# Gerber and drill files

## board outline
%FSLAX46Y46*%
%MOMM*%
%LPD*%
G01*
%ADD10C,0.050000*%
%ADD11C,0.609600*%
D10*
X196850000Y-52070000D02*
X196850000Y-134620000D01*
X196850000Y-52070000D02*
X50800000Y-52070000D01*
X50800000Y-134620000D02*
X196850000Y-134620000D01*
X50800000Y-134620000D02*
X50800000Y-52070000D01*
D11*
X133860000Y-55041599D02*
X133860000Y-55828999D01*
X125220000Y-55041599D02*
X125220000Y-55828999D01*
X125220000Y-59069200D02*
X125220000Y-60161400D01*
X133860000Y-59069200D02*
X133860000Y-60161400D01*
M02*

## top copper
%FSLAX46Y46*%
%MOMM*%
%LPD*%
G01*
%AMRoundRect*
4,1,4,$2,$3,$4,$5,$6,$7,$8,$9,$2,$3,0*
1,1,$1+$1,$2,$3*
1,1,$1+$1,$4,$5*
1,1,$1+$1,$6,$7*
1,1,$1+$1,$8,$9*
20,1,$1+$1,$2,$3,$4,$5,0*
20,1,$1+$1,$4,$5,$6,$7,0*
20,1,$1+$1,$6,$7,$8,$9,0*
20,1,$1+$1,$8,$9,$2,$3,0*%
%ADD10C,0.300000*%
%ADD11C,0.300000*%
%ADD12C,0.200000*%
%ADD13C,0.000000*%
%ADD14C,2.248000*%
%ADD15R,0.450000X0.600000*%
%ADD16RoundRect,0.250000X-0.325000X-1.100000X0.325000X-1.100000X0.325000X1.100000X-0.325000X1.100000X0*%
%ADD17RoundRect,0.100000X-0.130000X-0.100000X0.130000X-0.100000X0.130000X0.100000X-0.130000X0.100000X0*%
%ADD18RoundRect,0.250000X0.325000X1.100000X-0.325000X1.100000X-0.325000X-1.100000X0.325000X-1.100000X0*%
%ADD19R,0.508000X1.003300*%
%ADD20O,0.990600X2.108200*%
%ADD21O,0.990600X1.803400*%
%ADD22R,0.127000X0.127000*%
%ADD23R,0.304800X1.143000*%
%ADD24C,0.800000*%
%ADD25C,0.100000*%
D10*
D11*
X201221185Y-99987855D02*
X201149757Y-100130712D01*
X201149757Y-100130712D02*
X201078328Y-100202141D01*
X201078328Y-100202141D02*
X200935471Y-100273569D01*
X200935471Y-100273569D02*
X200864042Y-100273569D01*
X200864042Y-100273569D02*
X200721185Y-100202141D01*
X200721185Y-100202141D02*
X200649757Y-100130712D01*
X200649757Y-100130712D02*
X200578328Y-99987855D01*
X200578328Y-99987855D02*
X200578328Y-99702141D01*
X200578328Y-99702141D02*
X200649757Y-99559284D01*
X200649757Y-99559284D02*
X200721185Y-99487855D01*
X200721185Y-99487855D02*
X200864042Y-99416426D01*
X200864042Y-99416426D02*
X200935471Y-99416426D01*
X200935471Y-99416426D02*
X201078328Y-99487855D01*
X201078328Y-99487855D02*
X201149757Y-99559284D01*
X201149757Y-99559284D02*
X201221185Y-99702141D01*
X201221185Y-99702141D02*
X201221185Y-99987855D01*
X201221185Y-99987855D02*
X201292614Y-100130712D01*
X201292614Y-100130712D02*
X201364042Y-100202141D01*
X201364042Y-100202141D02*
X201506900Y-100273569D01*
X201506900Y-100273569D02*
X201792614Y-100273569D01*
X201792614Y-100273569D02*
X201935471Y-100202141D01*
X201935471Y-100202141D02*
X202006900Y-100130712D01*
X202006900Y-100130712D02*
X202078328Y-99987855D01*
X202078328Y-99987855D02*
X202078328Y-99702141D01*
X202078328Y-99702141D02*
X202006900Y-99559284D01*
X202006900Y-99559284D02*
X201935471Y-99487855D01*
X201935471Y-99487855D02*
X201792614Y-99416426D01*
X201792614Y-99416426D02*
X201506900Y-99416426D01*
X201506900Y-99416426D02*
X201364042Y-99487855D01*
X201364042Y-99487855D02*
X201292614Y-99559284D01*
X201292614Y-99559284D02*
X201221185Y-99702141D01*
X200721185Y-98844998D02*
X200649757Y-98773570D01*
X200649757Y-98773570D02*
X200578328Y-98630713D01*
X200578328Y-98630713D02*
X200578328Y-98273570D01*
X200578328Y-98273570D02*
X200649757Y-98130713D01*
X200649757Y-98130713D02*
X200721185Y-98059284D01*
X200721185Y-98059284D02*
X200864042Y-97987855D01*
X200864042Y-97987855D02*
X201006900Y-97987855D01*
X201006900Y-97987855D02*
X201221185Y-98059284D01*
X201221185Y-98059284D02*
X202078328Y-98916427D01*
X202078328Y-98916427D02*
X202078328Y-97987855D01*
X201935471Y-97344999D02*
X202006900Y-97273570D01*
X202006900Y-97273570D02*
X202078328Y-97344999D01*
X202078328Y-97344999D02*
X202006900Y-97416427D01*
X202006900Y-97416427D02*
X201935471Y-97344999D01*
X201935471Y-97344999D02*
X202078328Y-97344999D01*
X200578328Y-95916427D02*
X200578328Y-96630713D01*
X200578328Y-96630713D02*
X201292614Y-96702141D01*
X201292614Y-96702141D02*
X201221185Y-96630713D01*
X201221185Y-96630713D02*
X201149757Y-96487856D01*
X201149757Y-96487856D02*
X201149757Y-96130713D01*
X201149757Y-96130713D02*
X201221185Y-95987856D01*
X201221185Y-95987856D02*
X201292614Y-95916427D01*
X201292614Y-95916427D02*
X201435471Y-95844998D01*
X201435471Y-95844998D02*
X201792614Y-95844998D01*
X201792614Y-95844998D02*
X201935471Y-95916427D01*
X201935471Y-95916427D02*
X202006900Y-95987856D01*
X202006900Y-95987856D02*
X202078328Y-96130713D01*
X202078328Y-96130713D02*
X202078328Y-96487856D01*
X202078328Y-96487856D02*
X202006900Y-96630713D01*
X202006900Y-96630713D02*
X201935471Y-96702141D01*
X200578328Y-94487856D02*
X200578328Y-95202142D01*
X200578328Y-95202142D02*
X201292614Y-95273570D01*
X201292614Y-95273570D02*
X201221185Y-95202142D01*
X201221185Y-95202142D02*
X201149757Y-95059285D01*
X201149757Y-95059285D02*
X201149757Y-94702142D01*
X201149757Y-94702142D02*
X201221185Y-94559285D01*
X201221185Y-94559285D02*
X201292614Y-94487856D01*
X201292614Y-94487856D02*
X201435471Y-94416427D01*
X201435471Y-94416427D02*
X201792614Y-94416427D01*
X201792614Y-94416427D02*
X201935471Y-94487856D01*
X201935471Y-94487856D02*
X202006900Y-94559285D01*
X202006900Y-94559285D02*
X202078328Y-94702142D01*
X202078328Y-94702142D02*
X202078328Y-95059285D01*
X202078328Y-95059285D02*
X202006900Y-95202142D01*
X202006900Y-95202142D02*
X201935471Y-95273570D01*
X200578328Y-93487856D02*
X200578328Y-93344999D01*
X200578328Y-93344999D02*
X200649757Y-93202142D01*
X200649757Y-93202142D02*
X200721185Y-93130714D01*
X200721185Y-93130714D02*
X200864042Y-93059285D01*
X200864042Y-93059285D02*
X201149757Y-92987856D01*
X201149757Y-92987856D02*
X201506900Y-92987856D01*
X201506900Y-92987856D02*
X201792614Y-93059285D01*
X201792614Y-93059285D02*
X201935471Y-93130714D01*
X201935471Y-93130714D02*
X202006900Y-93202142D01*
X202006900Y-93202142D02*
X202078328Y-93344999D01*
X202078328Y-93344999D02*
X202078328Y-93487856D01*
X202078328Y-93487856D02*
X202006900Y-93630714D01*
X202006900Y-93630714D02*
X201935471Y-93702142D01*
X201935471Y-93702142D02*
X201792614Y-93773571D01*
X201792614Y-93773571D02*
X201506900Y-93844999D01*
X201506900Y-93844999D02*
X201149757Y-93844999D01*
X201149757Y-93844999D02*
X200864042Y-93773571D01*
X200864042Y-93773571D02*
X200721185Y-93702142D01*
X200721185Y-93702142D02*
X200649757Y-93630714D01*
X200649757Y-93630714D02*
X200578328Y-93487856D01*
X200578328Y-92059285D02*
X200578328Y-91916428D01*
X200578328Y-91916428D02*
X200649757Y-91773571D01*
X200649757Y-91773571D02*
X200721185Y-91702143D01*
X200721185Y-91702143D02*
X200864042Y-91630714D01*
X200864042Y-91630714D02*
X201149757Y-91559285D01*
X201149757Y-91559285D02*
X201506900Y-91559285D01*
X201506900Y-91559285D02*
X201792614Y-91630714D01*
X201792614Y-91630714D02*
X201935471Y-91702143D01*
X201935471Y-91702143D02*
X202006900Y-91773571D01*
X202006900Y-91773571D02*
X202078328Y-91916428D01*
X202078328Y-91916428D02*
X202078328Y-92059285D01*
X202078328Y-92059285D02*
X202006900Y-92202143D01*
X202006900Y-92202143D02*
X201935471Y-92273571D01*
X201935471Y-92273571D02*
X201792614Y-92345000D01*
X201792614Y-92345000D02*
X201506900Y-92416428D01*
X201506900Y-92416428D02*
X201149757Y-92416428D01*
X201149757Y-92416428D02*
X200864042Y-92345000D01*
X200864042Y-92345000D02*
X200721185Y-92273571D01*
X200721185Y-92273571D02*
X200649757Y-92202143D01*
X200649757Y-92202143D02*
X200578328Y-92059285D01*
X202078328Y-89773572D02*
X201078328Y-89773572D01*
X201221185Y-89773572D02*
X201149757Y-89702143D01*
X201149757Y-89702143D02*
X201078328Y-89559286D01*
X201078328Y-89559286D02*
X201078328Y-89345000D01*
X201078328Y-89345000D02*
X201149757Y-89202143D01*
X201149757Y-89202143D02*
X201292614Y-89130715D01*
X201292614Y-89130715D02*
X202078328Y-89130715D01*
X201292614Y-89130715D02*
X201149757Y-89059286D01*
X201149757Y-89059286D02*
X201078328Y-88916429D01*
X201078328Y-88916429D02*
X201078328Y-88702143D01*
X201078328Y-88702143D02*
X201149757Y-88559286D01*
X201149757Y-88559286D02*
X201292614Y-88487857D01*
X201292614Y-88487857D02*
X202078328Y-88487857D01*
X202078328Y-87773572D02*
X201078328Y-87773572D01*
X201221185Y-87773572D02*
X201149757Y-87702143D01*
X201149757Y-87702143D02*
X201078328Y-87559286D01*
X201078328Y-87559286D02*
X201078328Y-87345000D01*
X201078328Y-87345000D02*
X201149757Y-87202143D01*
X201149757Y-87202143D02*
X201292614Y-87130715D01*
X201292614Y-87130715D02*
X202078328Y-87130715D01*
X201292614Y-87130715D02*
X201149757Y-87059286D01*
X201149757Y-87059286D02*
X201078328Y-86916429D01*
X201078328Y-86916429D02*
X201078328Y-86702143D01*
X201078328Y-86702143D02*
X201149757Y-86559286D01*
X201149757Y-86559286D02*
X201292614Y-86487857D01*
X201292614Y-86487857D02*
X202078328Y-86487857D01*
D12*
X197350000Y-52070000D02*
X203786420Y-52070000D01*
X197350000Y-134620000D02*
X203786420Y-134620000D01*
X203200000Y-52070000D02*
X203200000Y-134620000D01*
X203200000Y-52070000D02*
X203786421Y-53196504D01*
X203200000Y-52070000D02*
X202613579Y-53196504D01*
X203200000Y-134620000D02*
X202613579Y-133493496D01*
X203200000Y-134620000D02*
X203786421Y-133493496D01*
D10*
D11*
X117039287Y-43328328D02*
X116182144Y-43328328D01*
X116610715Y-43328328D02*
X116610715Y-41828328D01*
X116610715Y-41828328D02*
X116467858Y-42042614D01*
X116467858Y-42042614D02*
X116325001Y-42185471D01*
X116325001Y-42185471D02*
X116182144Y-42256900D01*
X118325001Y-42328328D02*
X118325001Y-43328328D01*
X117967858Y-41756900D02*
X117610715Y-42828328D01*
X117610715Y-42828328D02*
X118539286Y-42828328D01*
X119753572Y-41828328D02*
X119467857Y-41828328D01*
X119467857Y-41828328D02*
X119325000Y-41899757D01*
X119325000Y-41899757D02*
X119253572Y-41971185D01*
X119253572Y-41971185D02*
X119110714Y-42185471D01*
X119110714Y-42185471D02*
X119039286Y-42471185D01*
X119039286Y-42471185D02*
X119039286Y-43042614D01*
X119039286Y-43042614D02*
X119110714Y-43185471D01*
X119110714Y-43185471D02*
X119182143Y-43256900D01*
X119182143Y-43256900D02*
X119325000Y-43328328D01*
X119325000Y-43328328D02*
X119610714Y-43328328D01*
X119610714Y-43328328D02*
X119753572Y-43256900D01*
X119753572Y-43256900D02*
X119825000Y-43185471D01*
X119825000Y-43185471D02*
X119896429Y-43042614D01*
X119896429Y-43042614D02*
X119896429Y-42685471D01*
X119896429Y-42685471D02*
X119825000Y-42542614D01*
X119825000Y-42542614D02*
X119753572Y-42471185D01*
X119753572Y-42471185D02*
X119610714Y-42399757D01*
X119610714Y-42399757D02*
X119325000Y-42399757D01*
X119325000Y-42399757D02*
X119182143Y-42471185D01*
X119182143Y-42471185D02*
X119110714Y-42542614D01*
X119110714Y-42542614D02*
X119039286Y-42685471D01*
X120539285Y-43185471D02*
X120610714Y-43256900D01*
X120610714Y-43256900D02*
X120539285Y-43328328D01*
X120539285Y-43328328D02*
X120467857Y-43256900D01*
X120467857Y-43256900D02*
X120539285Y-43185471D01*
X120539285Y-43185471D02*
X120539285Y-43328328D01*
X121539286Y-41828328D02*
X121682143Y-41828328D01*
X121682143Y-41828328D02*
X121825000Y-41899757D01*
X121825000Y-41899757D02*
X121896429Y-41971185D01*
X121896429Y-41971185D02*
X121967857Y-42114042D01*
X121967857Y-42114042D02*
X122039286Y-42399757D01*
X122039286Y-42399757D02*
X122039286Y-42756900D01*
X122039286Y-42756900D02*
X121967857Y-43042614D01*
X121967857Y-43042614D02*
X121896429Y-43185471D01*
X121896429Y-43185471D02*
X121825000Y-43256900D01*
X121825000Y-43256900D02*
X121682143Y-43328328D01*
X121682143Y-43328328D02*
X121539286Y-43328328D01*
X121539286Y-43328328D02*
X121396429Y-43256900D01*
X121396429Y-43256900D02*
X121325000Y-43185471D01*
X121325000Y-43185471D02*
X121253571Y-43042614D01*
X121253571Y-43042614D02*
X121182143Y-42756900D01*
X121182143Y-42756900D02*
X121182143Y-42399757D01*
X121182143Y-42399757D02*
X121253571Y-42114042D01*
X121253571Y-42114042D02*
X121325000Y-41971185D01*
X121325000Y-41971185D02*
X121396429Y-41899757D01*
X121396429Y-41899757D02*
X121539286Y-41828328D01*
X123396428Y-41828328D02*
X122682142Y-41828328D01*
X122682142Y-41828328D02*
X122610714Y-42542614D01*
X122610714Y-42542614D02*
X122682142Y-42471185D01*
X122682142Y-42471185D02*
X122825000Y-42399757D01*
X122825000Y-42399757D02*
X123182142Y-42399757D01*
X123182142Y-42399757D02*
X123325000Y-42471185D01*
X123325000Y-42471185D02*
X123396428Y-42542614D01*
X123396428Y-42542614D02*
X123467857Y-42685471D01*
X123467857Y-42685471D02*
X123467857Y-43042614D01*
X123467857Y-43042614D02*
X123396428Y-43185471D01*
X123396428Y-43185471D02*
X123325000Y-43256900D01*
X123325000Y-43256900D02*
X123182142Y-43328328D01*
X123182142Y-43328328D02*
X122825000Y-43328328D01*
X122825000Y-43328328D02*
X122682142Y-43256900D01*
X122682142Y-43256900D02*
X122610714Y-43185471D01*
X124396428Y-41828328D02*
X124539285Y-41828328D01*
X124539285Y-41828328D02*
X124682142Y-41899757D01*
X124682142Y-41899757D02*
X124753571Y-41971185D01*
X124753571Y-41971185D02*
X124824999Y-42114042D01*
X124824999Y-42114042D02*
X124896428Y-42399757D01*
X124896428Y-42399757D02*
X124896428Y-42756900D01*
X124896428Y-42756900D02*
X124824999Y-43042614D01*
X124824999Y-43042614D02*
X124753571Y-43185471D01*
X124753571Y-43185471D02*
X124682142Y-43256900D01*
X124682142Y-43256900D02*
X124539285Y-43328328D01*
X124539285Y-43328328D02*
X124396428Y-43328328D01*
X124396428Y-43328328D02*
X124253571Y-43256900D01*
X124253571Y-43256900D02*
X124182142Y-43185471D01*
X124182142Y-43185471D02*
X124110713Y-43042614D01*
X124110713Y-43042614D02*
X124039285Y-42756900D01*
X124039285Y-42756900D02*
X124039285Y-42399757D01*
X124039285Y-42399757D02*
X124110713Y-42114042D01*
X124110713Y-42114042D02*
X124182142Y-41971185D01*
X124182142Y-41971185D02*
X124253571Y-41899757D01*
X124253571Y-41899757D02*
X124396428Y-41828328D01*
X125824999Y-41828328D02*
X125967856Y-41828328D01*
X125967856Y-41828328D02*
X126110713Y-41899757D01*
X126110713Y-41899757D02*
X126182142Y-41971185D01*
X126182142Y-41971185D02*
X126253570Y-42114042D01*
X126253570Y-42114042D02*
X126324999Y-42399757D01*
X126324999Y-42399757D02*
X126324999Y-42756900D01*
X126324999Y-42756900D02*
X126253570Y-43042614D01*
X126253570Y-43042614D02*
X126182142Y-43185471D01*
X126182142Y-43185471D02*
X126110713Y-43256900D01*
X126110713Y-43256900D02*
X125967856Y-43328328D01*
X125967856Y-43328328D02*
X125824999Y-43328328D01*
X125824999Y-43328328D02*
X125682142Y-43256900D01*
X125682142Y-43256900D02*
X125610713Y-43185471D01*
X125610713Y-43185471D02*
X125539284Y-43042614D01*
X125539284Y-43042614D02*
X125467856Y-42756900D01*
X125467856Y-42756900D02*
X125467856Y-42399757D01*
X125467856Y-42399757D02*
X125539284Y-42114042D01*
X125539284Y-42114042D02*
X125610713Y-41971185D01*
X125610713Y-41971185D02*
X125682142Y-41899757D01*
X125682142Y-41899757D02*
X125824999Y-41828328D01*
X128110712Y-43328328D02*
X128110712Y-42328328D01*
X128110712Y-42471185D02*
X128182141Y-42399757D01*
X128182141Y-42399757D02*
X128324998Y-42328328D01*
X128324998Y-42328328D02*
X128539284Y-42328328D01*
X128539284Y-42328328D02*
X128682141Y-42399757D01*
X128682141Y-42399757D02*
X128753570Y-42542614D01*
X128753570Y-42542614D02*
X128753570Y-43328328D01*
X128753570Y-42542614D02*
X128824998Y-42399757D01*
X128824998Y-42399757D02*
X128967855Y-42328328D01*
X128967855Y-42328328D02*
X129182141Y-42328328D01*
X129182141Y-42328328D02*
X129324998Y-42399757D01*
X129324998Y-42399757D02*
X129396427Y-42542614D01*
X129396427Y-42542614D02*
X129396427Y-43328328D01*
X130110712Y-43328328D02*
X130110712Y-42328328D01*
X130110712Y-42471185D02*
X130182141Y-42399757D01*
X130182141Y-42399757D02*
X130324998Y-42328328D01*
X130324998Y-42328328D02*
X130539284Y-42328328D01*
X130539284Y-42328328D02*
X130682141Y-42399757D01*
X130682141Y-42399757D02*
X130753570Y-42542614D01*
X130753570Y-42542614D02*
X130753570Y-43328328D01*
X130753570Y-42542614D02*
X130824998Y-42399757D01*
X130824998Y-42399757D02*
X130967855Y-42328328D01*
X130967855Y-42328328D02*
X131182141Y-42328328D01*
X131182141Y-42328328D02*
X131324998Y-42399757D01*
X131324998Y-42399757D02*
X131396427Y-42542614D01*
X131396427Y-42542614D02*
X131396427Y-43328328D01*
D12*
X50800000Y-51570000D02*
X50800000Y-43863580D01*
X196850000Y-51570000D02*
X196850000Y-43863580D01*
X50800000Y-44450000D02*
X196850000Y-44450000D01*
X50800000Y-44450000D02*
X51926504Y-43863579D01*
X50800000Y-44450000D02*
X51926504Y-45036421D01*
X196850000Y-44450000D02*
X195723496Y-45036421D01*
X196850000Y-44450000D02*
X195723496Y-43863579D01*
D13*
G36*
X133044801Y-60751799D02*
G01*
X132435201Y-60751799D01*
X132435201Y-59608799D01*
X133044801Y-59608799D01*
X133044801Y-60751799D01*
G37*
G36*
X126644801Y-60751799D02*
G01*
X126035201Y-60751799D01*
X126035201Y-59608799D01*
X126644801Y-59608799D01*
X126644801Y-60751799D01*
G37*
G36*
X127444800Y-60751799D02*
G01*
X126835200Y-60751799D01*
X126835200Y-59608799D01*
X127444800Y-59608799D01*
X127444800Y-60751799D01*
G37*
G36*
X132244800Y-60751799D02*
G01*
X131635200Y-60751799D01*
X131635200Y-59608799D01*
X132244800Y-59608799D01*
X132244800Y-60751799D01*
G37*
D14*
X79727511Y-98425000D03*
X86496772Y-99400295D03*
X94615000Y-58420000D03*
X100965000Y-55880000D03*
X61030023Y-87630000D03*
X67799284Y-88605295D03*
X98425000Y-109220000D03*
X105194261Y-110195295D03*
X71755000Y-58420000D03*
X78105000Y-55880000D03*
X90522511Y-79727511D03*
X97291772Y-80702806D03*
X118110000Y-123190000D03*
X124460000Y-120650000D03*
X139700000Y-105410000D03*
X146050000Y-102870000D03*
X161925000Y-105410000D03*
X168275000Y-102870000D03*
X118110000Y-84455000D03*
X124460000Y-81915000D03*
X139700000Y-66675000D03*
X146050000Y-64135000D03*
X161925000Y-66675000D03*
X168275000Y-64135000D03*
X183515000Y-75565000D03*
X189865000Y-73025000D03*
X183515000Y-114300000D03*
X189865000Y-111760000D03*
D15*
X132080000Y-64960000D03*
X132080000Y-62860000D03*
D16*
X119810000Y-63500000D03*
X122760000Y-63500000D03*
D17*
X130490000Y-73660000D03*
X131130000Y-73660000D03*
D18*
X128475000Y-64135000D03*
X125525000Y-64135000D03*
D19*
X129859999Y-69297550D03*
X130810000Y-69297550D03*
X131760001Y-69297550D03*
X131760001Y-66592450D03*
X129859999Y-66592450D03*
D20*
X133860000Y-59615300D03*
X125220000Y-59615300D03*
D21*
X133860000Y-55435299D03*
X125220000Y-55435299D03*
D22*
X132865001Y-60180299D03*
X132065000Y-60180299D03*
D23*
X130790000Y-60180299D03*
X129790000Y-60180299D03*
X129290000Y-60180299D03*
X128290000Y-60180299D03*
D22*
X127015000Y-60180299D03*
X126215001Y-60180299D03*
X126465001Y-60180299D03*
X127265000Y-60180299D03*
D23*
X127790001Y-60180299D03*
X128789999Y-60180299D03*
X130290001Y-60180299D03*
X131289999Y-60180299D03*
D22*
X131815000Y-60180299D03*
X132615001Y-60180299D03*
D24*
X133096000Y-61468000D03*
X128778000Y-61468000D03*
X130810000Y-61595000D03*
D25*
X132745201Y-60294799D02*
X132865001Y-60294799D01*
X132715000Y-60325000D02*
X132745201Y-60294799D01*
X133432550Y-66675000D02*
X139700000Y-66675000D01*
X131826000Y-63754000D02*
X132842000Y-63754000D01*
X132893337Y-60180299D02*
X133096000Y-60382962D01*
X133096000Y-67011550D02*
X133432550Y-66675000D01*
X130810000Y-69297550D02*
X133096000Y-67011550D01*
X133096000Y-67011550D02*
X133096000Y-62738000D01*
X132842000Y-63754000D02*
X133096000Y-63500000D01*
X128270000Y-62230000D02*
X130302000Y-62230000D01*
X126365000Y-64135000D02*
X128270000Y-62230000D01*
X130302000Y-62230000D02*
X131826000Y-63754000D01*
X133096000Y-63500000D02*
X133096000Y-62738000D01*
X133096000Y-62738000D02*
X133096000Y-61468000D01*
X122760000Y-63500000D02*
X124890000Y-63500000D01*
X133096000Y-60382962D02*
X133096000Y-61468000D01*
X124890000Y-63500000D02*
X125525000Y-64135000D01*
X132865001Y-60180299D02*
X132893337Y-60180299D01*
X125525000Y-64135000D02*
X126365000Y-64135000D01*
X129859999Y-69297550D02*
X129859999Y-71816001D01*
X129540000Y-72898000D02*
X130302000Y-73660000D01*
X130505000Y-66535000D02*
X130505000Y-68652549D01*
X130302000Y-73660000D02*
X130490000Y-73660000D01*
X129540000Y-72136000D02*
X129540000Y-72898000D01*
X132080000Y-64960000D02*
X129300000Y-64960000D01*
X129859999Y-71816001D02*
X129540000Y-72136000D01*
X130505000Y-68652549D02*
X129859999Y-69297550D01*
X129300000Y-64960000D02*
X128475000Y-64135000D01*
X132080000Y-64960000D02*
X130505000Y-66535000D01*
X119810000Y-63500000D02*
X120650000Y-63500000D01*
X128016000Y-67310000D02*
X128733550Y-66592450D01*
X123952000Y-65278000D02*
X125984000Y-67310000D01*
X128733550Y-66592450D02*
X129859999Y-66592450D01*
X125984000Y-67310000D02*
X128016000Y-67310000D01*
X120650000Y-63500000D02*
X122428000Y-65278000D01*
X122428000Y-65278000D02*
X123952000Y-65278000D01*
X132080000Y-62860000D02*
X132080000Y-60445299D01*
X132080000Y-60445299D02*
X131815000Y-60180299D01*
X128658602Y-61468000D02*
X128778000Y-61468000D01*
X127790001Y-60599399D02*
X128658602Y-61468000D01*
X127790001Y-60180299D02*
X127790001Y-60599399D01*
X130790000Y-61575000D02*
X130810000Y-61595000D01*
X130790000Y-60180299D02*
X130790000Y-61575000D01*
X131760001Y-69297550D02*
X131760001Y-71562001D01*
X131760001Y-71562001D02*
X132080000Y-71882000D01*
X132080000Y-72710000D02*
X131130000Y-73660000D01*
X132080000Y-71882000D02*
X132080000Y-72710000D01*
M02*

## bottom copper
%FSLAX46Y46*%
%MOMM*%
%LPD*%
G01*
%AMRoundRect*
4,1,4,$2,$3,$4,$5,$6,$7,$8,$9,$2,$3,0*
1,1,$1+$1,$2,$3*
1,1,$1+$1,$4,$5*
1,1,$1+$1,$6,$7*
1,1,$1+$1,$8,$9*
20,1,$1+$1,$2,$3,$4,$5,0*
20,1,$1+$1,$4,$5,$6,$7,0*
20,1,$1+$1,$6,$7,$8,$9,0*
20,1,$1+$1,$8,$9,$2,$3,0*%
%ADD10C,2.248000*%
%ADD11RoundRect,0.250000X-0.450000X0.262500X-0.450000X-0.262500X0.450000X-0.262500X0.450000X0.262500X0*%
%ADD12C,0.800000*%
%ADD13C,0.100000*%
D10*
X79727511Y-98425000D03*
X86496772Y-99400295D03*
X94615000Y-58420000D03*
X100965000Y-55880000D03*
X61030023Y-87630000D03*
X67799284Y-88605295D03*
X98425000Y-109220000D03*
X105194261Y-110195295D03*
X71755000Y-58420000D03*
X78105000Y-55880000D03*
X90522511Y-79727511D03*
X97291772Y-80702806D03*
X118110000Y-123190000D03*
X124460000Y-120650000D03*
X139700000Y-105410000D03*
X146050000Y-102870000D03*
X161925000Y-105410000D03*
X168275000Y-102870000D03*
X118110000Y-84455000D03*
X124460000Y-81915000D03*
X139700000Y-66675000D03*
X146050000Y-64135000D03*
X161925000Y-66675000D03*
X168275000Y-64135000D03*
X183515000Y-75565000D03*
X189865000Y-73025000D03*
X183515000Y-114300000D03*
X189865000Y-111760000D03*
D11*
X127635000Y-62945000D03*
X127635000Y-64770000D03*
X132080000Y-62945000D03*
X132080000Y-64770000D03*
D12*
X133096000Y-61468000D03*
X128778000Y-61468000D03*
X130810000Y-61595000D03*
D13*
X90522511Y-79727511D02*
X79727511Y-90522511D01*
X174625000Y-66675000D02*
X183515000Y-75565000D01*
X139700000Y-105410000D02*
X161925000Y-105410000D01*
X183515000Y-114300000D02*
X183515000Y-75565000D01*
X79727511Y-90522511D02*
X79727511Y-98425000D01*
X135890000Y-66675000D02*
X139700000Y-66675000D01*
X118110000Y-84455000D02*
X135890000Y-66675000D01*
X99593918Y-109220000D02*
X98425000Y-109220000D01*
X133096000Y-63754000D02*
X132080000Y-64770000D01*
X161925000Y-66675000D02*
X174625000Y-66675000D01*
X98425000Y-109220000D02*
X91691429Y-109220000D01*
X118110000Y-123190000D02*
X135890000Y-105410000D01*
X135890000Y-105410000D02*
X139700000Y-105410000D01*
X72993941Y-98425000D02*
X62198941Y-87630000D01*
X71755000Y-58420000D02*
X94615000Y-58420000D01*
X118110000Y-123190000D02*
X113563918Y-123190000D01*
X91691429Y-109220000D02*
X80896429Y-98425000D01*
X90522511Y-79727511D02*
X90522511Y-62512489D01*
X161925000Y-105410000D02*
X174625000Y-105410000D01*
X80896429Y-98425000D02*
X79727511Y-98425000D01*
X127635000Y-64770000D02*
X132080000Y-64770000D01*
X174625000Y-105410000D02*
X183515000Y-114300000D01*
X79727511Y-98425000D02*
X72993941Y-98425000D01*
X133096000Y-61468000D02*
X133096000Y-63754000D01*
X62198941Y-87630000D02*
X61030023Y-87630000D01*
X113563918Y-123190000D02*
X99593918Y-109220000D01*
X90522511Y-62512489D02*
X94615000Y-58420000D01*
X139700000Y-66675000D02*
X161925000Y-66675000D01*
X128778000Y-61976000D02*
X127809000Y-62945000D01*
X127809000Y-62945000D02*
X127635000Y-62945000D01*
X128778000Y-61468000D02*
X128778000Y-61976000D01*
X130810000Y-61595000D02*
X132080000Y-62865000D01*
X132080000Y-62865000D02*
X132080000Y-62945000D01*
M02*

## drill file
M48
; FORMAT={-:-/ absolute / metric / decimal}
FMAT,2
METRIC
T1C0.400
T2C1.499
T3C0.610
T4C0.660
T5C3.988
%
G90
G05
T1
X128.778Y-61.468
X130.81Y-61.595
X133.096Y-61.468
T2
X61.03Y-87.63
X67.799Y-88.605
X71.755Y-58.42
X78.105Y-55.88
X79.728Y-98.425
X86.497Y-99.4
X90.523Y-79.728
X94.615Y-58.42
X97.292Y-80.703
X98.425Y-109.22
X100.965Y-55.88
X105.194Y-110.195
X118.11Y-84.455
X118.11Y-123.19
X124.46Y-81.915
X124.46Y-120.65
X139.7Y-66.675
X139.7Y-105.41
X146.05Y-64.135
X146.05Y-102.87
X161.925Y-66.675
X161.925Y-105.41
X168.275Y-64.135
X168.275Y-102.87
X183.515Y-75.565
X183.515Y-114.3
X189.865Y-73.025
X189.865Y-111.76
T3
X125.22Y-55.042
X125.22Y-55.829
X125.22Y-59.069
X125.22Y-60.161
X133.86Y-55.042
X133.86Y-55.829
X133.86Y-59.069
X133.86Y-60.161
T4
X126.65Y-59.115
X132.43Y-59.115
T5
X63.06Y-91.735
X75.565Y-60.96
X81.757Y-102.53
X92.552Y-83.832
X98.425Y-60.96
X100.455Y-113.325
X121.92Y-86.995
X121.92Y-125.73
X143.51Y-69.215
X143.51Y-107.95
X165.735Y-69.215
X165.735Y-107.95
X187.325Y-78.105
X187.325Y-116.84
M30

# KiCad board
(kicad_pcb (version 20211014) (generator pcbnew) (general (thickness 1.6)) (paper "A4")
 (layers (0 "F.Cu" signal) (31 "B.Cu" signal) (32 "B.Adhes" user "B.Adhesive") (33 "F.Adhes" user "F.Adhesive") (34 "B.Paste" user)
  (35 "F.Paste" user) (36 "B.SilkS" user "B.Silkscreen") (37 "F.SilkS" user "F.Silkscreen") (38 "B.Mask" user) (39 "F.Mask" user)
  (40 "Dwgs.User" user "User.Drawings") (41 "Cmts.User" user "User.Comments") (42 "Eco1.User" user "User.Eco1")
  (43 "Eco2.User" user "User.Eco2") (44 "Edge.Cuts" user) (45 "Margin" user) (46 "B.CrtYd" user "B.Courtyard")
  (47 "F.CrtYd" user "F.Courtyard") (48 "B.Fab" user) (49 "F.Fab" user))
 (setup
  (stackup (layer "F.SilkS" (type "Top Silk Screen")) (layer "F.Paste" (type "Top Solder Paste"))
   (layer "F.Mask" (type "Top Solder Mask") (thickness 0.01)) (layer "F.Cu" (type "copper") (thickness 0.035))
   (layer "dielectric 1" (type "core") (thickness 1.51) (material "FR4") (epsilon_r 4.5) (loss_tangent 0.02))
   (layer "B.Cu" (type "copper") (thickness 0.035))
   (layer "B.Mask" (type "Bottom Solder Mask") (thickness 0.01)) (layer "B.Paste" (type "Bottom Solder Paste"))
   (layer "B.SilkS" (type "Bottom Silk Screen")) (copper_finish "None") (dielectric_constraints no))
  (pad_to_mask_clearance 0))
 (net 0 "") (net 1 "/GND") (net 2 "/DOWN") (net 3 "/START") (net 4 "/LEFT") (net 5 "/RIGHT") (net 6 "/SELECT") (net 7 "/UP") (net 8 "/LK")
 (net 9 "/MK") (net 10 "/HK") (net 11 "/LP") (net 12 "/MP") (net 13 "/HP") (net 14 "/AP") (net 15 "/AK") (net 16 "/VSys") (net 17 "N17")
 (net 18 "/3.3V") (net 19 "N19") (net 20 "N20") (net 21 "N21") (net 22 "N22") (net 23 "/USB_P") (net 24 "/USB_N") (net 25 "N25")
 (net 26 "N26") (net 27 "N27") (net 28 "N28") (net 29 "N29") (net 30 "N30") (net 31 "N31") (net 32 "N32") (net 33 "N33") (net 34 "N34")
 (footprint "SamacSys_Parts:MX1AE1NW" (layer "F.Cu") (at 79.727511 98.425 -30)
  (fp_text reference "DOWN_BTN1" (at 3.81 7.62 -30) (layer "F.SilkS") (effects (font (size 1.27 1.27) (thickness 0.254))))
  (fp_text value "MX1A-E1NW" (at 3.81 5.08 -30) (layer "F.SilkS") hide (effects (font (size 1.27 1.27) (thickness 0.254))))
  (pad "" np_thru_hole circle (at 3.81 2.54 330) (size 3.9878 3.9878) (drill 3.9878) (layers *.Cu *.Mask))
  (pad "1" thru_hole circle (at 0 0 330) (size 2.248 2.248) (drill 1.4986) (layers *.Cu *.Mask) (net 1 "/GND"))
  (pad "2" thru_hole circle (at 6.35 -2.54 330) (size 2.248 2.248) (drill 1.4986) (layers *.Cu *.Mask) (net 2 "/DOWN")))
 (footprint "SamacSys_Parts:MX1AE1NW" (layer "F.Cu") (at 94.615 58.42)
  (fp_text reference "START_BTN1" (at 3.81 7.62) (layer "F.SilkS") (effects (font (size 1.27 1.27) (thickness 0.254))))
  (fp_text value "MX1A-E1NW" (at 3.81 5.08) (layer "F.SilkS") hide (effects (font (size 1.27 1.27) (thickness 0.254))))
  (pad "" np_thru_hole circle (at 3.81 2.54) (size 3.9878 3.9878) (drill 3.9878) (layers *.Cu *.Mask))
  (pad "1" thru_hole circle (at 0 0) (size 2.248 2.248) (drill 1.4986) (layers *.Cu *.Mask) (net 1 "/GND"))
  (pad "2" thru_hole circle (at 6.35 -2.54) (size 2.248 2.248) (drill 1.4986) (layers *.Cu *.Mask) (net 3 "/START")))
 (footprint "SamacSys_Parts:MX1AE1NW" (layer "F.Cu") (at 61.030023 87.63 -30)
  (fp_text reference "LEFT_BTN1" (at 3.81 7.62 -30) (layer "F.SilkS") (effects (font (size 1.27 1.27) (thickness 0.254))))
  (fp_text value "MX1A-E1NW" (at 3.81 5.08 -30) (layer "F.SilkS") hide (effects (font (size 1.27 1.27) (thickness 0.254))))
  (pad "" np_thru_hole circle (at 3.81 2.54 330) (size 3.9878 3.9878) (drill 3.9878) (layers *.Cu *.Mask))
  (pad "1" thru_hole circle (at 0 0 330) (size 2.248 2.248) (drill 1.4986) (layers *.Cu *.Mask) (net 1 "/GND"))
  (pad "2" thru_hole circle (at 6.35 -2.54 330) (size 2.248 2.248) (drill 1.4986) (layers *.Cu *.Mask) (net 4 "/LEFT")))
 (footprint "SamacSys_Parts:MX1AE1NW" (layer "F.Cu") (at 98.425 109.22 -30)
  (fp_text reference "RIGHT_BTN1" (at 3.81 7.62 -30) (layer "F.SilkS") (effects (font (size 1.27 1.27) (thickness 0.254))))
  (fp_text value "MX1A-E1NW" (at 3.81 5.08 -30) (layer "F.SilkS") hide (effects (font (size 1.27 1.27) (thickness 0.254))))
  (pad "" np_thru_hole circle (at 3.81 2.54 330) (size 3.9878 3.9878) (drill 3.9878) (layers *.Cu *.Mask))
  (pad "1" thru_hole circle (at 0 0 330) (size 2.248 2.248) (drill 1.4986) (layers *.Cu *.Mask) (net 1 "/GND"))
  (pad "2" thru_hole circle (at 6.35 -2.54 330) (size 2.248 2.248) (drill 1.4986) (layers *.Cu *.Mask) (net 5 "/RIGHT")))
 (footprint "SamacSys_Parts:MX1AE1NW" (layer "F.Cu") (at 71.755 58.42)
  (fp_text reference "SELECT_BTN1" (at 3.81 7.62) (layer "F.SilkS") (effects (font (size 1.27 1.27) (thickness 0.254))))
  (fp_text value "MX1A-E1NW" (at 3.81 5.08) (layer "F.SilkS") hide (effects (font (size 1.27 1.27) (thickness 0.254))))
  (pad "" np_thru_hole circle (at 3.81 2.54) (size 3.9878 3.9878) (drill 3.9878) (layers *.Cu *.Mask))
  (pad "1" thru_hole circle (at 0 0) (size 2.248 2.248) (drill 1.4986) (layers *.Cu *.Mask) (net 1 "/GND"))
  (pad "2" thru_hole circle (at 6.35 -2.54) (size 2.248 2.248) (drill 1.4986) (layers *.Cu *.Mask) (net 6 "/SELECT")))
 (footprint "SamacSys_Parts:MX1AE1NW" (layer "F.Cu") (at 90.522511 79.727511 -30)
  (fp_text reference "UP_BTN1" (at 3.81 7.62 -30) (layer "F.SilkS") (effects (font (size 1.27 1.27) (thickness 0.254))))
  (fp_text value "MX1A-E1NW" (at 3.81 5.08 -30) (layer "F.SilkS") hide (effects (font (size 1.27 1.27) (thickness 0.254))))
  (pad "" np_thru_hole circle (at 3.81 2.54 330) (size 3.9878 3.9878) (drill 3.9878) (layers *.Cu *.Mask))
  (pad "1" thru_hole circle (at 0 0 330) (size 2.248 2.248) (drill 1.4986) (layers *.Cu *.Mask) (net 1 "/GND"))
  (pad "2" thru_hole circle (at 6.35 -2.54 330) (size 2.248 2.248) (drill 1.4986) (layers *.Cu *.Mask) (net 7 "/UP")))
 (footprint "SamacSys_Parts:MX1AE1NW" (layer "F.Cu") (at 118.11 123.19)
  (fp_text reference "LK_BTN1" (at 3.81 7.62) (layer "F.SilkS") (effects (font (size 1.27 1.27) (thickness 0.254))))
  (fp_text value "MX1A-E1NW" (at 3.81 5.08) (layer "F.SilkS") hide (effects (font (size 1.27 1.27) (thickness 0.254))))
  (pad "" np_thru_hole circle (at 3.81 2.54) (size 3.9878 3.9878) (drill 3.9878) (layers *.Cu *.Mask))
  (pad "1" thru_hole circle (at 0 0) (size 2.248 2.248) (drill 1.4986) (layers *.Cu *.Mask) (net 1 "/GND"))
  (pad "2" thru_hole circle (at 6.35 -2.54) (size 2.248 2.248) (drill 1.4986) (layers *.Cu *.Mask) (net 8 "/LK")))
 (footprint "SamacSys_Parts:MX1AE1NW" (layer "F.Cu") (at 139.7 105.41)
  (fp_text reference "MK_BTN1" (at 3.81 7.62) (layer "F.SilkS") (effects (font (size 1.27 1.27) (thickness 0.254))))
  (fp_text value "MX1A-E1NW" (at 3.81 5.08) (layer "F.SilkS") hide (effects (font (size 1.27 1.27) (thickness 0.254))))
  (pad "" np_thru_hole circle (at 3.81 2.54) (size 3.9878 3.9878) (drill 3.9878) (layers *.Cu *.Mask))
  (pad "1" thru_hole circle (at 0 0) (size 2.248 2.248) (drill 1.4986) (layers *.Cu *.Mask) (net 1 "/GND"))
  (pad "2" thru_hole circle (at 6.35 -2.54) (size 2.248 2.248) (drill 1.4986) (layers *.Cu *.Mask) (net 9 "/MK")))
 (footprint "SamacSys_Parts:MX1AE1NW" (layer "F.Cu") (at 161.925 105.41)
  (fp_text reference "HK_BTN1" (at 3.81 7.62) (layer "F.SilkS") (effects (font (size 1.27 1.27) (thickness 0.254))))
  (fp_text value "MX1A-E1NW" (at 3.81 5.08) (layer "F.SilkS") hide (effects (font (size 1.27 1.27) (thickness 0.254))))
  (pad "" np_thru_hole circle (at 3.81 2.54) (size 3.9878 3.9878) (drill 3.9878) (layers *.Cu *.Mask))
  (pad "1" thru_hole circle (at 0 0) (size 2.248 2.248) (drill 1.4986) (layers *.Cu *.Mask) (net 1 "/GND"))
  (pad "2" thru_hole circle (at 6.35 -2.54) (size 2.248 2.248) (drill 1.4986) (layers *.Cu *.Mask) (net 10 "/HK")))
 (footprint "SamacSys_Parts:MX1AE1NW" (layer "F.Cu") (at 118.11 84.455)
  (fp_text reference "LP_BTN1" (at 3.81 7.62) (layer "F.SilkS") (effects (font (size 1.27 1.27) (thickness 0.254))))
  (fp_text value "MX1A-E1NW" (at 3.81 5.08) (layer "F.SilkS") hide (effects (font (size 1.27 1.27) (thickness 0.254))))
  (pad "" np_thru_hole circle (at 3.81 2.54) (size 3.9878 3.9878) (drill 3.9878) (layers *.Cu *.Mask))
  (pad "1" thru_hole circle (at 0 0) (size 2.248 2.248) (drill 1.4986) (layers *.Cu *.Mask) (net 1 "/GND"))
  (pad "2" thru_hole circle (at 6.35 -2.54) (size 2.248 2.248) (drill 1.4986) (layers *.Cu *.Mask) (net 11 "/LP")))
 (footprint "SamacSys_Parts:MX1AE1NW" (layer "F.Cu") (at 139.7 66.675)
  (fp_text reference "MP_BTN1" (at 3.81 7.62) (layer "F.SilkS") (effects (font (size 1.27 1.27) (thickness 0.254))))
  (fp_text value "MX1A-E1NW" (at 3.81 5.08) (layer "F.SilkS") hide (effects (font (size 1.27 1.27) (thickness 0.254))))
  (pad "" np_thru_hole circle (at 3.81 2.54) (size 3.9878 3.9878) (drill 3.9878) (layers *.Cu *.Mask))
  (pad "1" thru_hole circle (at 0 0) (size 2.248 2.248) (drill 1.4986) (layers *.Cu *.Mask) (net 1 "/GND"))
  (pad "2" thru_hole circle (at 6.35 -2.54) (size 2.248 2.248) (drill 1.4986) (layers *.Cu *.Mask) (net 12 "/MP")))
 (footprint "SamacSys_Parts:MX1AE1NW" (layer "F.Cu") (at 161.925 66.675)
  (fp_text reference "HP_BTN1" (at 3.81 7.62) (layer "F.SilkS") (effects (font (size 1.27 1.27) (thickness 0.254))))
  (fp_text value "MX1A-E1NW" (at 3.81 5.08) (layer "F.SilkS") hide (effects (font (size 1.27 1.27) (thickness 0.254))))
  (pad "" np_thru_hole circle (at 3.81 2.54) (size 3.9878 3.9878) (drill 3.9878) (layers *.Cu *.Mask))
  (pad "1" thru_hole circle (at 0 0) (size 2.248 2.248) (drill 1.4986) (layers *.Cu *.Mask) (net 1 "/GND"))
  (pad "2" thru_hole circle (at 6.35 -2.54) (size 2.248 2.248) (drill 1.4986) (layers *.Cu *.Mask) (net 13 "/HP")))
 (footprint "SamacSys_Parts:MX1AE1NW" (layer "F.Cu") (at 183.515 75.565)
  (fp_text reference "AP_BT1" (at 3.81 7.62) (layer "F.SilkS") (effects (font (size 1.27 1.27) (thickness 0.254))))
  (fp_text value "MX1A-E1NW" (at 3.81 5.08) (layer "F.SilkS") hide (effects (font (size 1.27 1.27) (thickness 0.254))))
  (pad "" np_thru_hole circle (at 3.81 2.54) (size 3.9878 3.9878) (drill 3.9878) (layers *.Cu *.Mask))
  (pad "1" thru_hole circle (at 0 0) (size 2.248 2.248) (drill 1.4986) (layers *.Cu *.Mask) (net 1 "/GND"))
  (pad "2" thru_hole circle (at 6.35 -2.54) (size 2.248 2.248) (drill 1.4986) (layers *.Cu *.Mask) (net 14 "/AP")))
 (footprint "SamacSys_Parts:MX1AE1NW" (layer "F.Cu") (at 183.515 114.3)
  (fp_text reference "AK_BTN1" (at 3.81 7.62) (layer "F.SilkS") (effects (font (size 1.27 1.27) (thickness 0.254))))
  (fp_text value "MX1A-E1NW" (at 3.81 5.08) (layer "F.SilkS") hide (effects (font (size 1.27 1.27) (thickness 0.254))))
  (pad "" np_thru_hole circle (at 3.81 2.54) (size 3.9878 3.9878) (drill 3.9878) (layers *.Cu *.Mask))
  (pad "1" thru_hole circle (at 0 0) (size 2.248 2.248) (drill 1.4986) (layers *.Cu *.Mask) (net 1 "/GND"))
  (pad "2" thru_hole circle (at 6.35 -2.54) (size 2.248 2.248) (drill 1.4986) (layers *.Cu *.Mask) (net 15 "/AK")))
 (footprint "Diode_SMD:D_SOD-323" (layer "F.Cu") (at 132.08 63.91 90)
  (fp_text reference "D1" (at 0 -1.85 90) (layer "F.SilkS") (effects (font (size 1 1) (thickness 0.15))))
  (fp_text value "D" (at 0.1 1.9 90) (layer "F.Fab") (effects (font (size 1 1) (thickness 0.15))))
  (pad "1" smd rect (at -1.05 0 90) (size 0.6 0.45) (layers "F.Cu" "F.Paste" "F.Mask") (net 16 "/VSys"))
  (pad "2" smd rect (at 1.05 0 90) (size 0.6 0.45) (layers "F.Cu" "F.Paste" "F.Mask") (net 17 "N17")))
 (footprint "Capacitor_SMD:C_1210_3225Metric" (layer "F.Cu") (at 121.285 63.5)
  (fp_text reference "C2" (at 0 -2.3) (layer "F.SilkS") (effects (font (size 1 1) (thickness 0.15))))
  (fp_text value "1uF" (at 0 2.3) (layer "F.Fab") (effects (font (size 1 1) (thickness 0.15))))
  (pad "1" smd roundrect (at -1.475 0) (size 1.15 2.7) (layers "F.Cu" "F.Paste" "F.Mask") (roundrect_rratio 0.217391) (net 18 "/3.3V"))
  (pad "2" smd roundrect (at 1.475 0) (size 1.15 2.7) (layers "F.Cu" "F.Paste" "F.Mask") (roundrect_rratio 0.217391) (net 1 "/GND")))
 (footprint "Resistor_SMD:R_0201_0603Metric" (layer "F.Cu") (at 130.81 73.66)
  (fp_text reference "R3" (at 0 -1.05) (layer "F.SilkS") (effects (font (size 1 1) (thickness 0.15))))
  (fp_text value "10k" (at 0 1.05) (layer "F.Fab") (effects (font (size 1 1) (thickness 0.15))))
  (pad "" smd roundrect (at -0.345 0) (size 0.318 0.36) (layers "F.Paste") (roundrect_rratio 0.25))
  (pad "" smd roundrect (at 0.345 0) (size 0.318 0.36) (layers "F.Paste") (roundrect_rratio 0.25))
  (pad "1" smd roundrect (at -0.32 0) (size 0.46 0.4) (layers "F.Cu" "F.Mask") (roundrect_rratio 0.25) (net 16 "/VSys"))
  (pad "2" smd roundrect (at 0.32 0) (size 0.46 0.4) (layers "F.Cu" "F.Mask") (roundrect_rratio 0.25) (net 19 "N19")))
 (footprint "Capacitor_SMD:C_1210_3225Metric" (layer "F.Cu") (at 127 64.135 180)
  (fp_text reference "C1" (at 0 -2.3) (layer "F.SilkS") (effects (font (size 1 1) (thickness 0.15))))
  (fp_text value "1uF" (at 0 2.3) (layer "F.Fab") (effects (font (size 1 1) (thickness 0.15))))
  (pad "1" smd roundrect (at -1.475 0 180) (size 1.15 2.7) (layers "F.Cu" "F.Paste" "F.Mask") (roundrect_rratio 0.217391) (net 16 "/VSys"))
  (pad "2" smd roundrect (at 1.475 0 180) (size 1.15 2.7) (layers "F.Cu" "F.Paste" "F.Mask") (roundrect_rratio 0.217391) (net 1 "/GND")))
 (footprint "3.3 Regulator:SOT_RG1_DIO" (layer "F.Cu") (at 130.81 67.945 90)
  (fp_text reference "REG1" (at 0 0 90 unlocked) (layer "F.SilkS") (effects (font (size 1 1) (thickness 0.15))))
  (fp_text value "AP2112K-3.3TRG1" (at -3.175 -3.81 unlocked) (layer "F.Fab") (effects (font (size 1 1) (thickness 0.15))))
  (pad "1" smd rect (at -1.35255 -0.950001 90) (size 1.0033 0.508) (layers "F.Cu" "F.Paste" "F.Mask") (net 16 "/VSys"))
  (pad "2" smd rect (at -1.35255 0 90) (size 1.0033 0.508) (layers "F.Cu" "F.Paste" "F.Mask") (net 1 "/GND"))
  (pad "3" smd rect (at -1.35255 0.950001 90) (size 1.0033 0.508) (layers "F.Cu" "F.Paste" "F.Mask") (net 19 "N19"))
  (pad "4" smd rect (at 1.35255 0.950001 90) (size 1.0033 0.508) (layers "F.Cu" "F.Paste" "F.Mask") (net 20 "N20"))
  (pad "5" smd rect (at 1.35255 -0.950001 90) (size 1.0033 0.508) (layers "F.Cu" "F.Paste" "F.Mask") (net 18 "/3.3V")))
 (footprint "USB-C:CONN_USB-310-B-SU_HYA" (layer "F.Cu") (at 129.54 56.515 180)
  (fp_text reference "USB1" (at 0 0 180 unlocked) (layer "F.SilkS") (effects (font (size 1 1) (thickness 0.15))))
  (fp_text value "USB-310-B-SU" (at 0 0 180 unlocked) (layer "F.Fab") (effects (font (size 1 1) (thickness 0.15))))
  (fp_poly
   (pts (xy -2.895201 -4.236799) (xy -3.504801 -4.236799) (xy -3.504801 -3.093799) (xy -2.895201 -3.093799)) (layer "F.Cu") (width 0)
   (fill solid))
  (fp_poly
   (pts (xy 3.504799 -4.236799) (xy 2.895199 -4.236799) (xy 2.895199 -3.093799) (xy 3.504799 -3.093799)) (layer "F.Cu") (width 0)
   (fill solid))
  (fp_poly
   (pts (xy 2.7048 -4.236799) (xy 2.0952 -4.236799) (xy 2.0952 -3.093799) (xy 2.7048 -3.093799)) (layer "F.Cu") (width 0) (fill solid))
  (fp_poly
   (pts (xy -2.0952 -4.236799) (xy -2.7048 -4.236799) (xy -2.7048 -3.093799) (xy -2.0952 -3.093799)) (layer "F.Cu") (width 0) (fill solid))
  (fp_line (start -4.32 1.473401) (end -4.32 0.686001) (layer "Edge.Cuts") (width 0.6096))
  (fp_line (start 4.32 1.473401) (end 4.32 0.686001) (layer "Edge.Cuts") (width 0.6096))
  (fp_line (start 4.32 -2.5542) (end 4.32 -3.6464) (layer "Edge.Cuts") (width 0.6096))
  (fp_line (start -4.32 -2.5542) (end -4.32 -3.6464) (layer "Edge.Cuts") (width 0.6096))
  (pad "" np_thru_hole circle (at -4.32 1.473401 180) (size 0.6096 0.6096) (drill 0.6096) (layers))
  (pad "" np_thru_hole circle (at 4.32 0.686001 180) (size 0.6096 0.6096) (drill 0.6096) (layers))
  (pad "" np_thru_hole circle (at 2.889999 -2.6003 180) (size 0.6604 0.6604) (drill 0.6604) (layers *.Cu *.Mask))
  (pad "" np_thru_hole circle (at -4.32 0.686001 180) (size 0.6096 0.6096) (drill 0.6096) (layers))
  (pad "" np_thru_hole circle (at -2.889999 -2.6003 180) (size 0.6604 0.6604) (drill 0.6604) (layers *.Cu *.Mask))
  (pad "" np_thru_hole circle (at -4.32 -2.5542 180) (size 0.6096 0.6096) (drill 0.6096) (layers))
  (pad "" np_thru_hole circle (at -4.32 -3.6464 180) (size 0.6096 0.6096) (drill 0.6096) (layers))
  (pad "" np_thru_hole circle (at 4.32 1.473401 180) (size 0.6096 0.6096) (drill 0.6096) (layers))
  (pad "" np_thru_hole circle (at 4.32 -3.6464 180) (size 0.6096 0.6096) (drill 0.6096) (layers))
  (pad "" np_thru_hole circle (at 4.32 -2.5542 180) (size 0.6096 0.6096) (drill 0.6096) (layers))
  (pad "19" smd oval (at -4.32 -3.1003 180) (size 0.9906 2.1082) (layers "F.Cu" "F.Paste" "F.Mask"))
  (pad "20" smd oval (at 4.32 -3.1003 180) (size 0.9906 2.1082) (layers "F.Cu" "F.Paste" "F.Mask"))
  (pad "21" smd oval (at -4.32 1.079701 180) (size 0.9906 1.8034) (layers "F.Cu" "F.Paste" "F.Mask"))
  (pad "22" smd oval (at 4.32 1.079701 180) (size 0.9906 1.8034) (layers "F.Cu" "F.Paste" "F.Mask"))
  (pad "A1" smd rect (at -3.325001 -3.665299 180) (size 0.127 0.127) (layers "F.Cu" "F.Paste" "F.Mask") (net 1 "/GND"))
  (pad "A4" smd rect (at -2.525 -3.665299 180) (size 0.127 0.127) (layers "F.Cu" "F.Paste" "F.Mask") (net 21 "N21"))
  (pad "A5" smd rect (at -1.25 -3.665299 180) (size 0.3048 1.143) (layers "F.Cu" "F.Paste" "F.Mask") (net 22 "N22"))
  (pad "A6" smd rect (at -0.25 -3.665299 180) (size 0.3048 1.143) (layers "F.Cu" "F.Paste" "F.Mask") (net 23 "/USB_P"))
  (pad "A7" smd rect (at 0.25 -3.665299 180) (size 0.3048 1.143) (layers "F.Cu" "F.Paste" "F.Mask") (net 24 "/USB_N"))
  (pad "A8" smd rect (at 1.25 -3.665299 180) (size 0.3048 1.143) (layers "F.Cu" "F.Paste" "F.Mask") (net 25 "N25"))
  (pad "A9" smd rect (at 2.525 -3.665299 180) (size 0.127 0.127) (layers "F.Cu" "F.Paste" "F.Mask") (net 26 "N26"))
  (pad "A12" smd rect (at 3.324999 -3.665299 180) (size 0.127 0.127) (layers "F.Cu" "F.Paste" "F.Mask") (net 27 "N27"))
  (pad "B1" smd rect (at 3.074999 -3.665299 180) (size 0.127 0.127) (layers "F.Cu" "F.Paste" "F.Mask") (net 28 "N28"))
  (pad "B4" smd rect (at 2.275 -3.665299 180) (size 0.127 0.127) (layers "F.Cu" "F.Paste" "F.Mask") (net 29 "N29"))
  (pad "B5" smd rect (at 1.749999 -3.665299 180) (size 0.3048 1.143) (layers "F.Cu" "F.Paste" "F.Mask") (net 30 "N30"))
  (pad "B6" smd rect (at 0.750001 -3.665299 180) (size 0.3048 1.143) (layers "F.Cu" "F.Paste" "F.Mask") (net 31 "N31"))
  (pad "B7" smd rect (at -0.750001 -3.665299 180) (size 0.3048 1.143) (layers "F.Cu" "F.Paste" "F.Mask") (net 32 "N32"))
  (pad "B8" smd rect (at -1.749999 -3.665299 180) (size 0.3048 1.143) (layers "F.Cu" "F.Paste" "F.Mask") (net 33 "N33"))
  (pad "B9" smd rect (at -2.275 -3.665299 180) (size 0.127 0.127) (layers "F.Cu" "F.Paste" "F.Mask") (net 17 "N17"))
  (pad "B12" smd rect (at -3.075001 -3.665299 180) (size 0.127 0.127) (layers "F.Cu" "F.Paste" "F.Mask") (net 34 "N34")))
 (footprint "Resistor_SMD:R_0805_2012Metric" (layer "B.Cu") (at 127.635 63.8575 -90)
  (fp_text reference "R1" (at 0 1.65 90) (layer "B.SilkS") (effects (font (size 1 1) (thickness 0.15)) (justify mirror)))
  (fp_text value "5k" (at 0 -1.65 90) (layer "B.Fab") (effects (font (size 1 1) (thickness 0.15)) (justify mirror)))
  (pad "1" smd roundrect (at -0.9125 0 270) (size 1.025 1.4) (layers "B.Cu" "B.Paste" "B.Mask") (roundrect_rratio 0.243902) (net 30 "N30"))
  (pad "2" smd roundrect (at 0.9125 0 270) (size 1.025 1.4) (layers "B.Cu" "B.Paste" "B.Mask") (roundrect_rratio 0.243902) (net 1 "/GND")))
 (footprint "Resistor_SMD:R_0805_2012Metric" (layer "B.Cu") (at 132.08 63.8575 -90)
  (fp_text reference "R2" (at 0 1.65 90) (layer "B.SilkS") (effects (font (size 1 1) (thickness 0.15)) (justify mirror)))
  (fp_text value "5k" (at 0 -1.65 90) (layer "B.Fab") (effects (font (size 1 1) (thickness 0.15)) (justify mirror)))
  (pad "1" smd roundrect (at -0.9125 0 270) (size 1.025 1.4) (layers "B.Cu" "B.Paste" "B.Mask") (roundrect_rratio 0.243902) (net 22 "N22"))
  (pad "2" smd roundrect (at 0.9125 0 270) (size 1.025 1.4) (layers "B.Cu" "B.Paste" "B.Mask") (roundrect_rratio 0.243902) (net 1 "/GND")))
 (gr_line (start 196.85 52.07) (end 196.85 134.62) (layer "Edge.Cuts") (width 0.05))
 (gr_line (start 196.85 52.07) (end 50.8 52.07) (layer "Edge.Cuts") (width 0.05))
 (gr_line (start 50.8 134.62) (end 196.85 134.62) (layer "Edge.Cuts") (width 0.05))
 (gr_line (start 50.8 134.62) (end 50.8 52.07) (layer "Edge.Cuts") (width 0.05))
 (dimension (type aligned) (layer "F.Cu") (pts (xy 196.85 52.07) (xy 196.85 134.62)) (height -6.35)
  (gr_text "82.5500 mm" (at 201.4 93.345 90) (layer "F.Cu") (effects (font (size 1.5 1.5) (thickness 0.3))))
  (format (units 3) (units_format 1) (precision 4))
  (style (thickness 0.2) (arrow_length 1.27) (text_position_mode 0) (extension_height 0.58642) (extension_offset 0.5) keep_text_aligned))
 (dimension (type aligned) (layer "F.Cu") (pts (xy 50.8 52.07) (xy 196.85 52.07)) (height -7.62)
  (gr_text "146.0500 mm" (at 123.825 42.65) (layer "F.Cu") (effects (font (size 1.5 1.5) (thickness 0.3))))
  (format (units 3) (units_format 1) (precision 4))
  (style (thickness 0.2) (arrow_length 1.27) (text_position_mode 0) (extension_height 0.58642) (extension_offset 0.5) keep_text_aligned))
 (segment (start 132.745201 60.294799) (end 132.865001 60.294799) (width 0.1) (layer "F.Cu") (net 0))
 (segment (start 132.715 60.325) (end 132.745201 60.294799) (width 0.1) (layer "F.Cu") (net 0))
 (segment (start 133.43255 66.675) (end 139.7 66.675) (width 0.1) (layer "F.Cu") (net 1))
 (segment (start 131.826 63.754) (end 132.842 63.754) (width 0.1) (layer "F.Cu") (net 1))
 (segment (start 132.893337 60.180299) (end 133.096 60.382962) (width 0.1) (layer "F.Cu") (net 1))
 (segment (start 133.096 67.01155) (end 133.43255 66.675) (width 0.1) (layer "F.Cu") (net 1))
 (segment (start 130.81 69.29755) (end 133.096 67.01155) (width 0.1) (layer "F.Cu") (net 1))
 (segment (start 133.096 67.01155) (end 133.096 62.738) (width 0.1) (layer "F.Cu") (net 1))
 (segment (start 132.842 63.754) (end 133.096 63.5) (width 0.1) (layer "F.Cu") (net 1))
 (segment (start 128.27 62.23) (end 130.302 62.23) (width 0.1) (layer "F.Cu") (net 1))
 (segment (start 126.365 64.135) (end 128.27 62.23) (width 0.1) (layer "F.Cu") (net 1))
 (segment (start 130.302 62.23) (end 131.826 63.754) (width 0.1) (layer "F.Cu") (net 1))
 (segment (start 133.096 63.5) (end 133.096 62.738) (width 0.1) (layer "F.Cu") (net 1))
 (segment (start 133.096 62.738) (end 133.096 61.468) (width 0.1) (layer "F.Cu") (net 1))
 (segment (start 122.76 63.5) (end 124.89 63.5) (width 0.1) (layer "F.Cu") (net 1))
 (segment (start 133.096 60.382962) (end 133.096 61.468) (width 0.1) (layer "F.Cu") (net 1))
 (segment (start 124.89 63.5) (end 125.525 64.135) (width 0.1) (layer "F.Cu") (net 1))
 (segment (start 132.865001 60.180299) (end 132.893337 60.180299) (width 0.1) (layer "F.Cu") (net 1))
 (segment (start 125.525 64.135) (end 126.365 64.135) (width 0.1) (layer "F.Cu") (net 1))
 (via (at 133.096 61.468) (size 0.8) (drill 0.4) (layers "F.Cu" "B.Cu") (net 1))
 (segment (start 90.522511 79.727511) (end 79.727511 90.522511) (width 0.1) (layer "B.Cu") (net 1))
 (segment (start 174.625 66.675) (end 183.515 75.565) (width 0.1) (layer "B.Cu") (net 1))
 (segment (start 139.7 105.41) (end 161.925 105.41) (width 0.1) (layer "B.Cu") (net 1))
 (segment (start 183.515 114.3) (end 183.515 75.565) (width 0.1) (layer "B.Cu") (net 1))
 (segment (start 79.727511 90.522511) (end 79.727511 98.425) (width 0.1) (layer "B.Cu") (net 1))
 (segment (start 135.89 66.675) (end 139.7 66.675) (width 0.1) (layer "B.Cu") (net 1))
 (segment (start 118.11 84.455) (end 135.89 66.675) (width 0.1) (layer "B.Cu") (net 1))
 (segment (start 99.593918 109.22) (end 98.425 109.22) (width 0.1) (layer "B.Cu") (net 1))
 (segment (start 133.096 63.754) (end 132.08 64.77) (width 0.1) (layer "B.Cu") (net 1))
 (segment (start 161.925 66.675) (end 174.625 66.675) (width 0.1) (layer "B.Cu") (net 1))
 (segment (start 98.425 109.22) (end 91.691429 109.22) (width 0.1) (layer "B.Cu") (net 1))
 (segment (start 118.11 123.19) (end 135.89 105.41) (width 0.1) (layer "B.Cu") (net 1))
 (segment (start 135.89 105.41) (end 139.7 105.41) (width 0.1) (layer "B.Cu") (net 1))
 (segment (start 72.993941 98.425) (end 62.198941 87.63) (width 0.1) (layer "B.Cu") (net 1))
 (segment (start 71.755 58.42) (end 94.615 58.42) (width 0.1) (layer "B.Cu") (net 1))
 (segment (start 118.11 123.19) (end 113.563918 123.19) (width 0.1) (layer "B.Cu") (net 1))
 (segment (start 91.691429 109.22) (end 80.896429 98.425) (width 0.1) (layer "B.Cu") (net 1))
 (segment (start 90.522511 79.727511) (end 90.522511 62.512489) (width 0.1) (layer "B.Cu") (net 1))
 (segment (start 161.925 105.41) (end 174.625 105.41) (width 0.1) (layer "B.Cu") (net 1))
 (segment (start 80.896429 98.425) (end 79.727511 98.425) (width 0.1) (layer "B.Cu") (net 1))
 (segment (start 127.635 64.77) (end 132.08 64.77) (width 0.1) (layer "B.Cu") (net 1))
 (segment (start 174.625 105.41) (end 183.515 114.3) (width 0.1) (layer "B.Cu") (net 1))
 (segment (start 79.727511 98.425) (end 72.993941 98.425) (width 0.1) (layer "B.Cu") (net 1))
 (segment (start 133.096 61.468) (end 133.096 63.754) (width 0.1) (layer "B.Cu") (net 1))
 (segment (start 62.198941 87.63) (end 61.030023 87.63) (width 0.1) (layer "B.Cu") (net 1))
 (segment (start 113.563918 123.19) (end 99.593918 109.22) (width 0.1) (layer "B.Cu") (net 1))
 (segment (start 90.522511 62.512489) (end 94.615 58.42) (width 0.1) (layer "B.Cu") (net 1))
 (segment (start 139.7 66.675) (end 161.925 66.675) (width 0.1) (layer "B.Cu") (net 1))
 (segment (start 129.859999 69.29755) (end 129.859999 71.816001) (width 0.1) (layer "F.Cu") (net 16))
 (segment (start 129.54 72.898) (end 130.302 73.66) (width 0.1) (layer "F.Cu") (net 16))
 (segment (start 130.505 66.535) (end 130.505 68.652549) (width 0.1) (layer "F.Cu") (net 16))
 (segment (start 130.302 73.66) (end 130.49 73.66) (width 0.1) (layer "F.Cu") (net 16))
 (segment (start 129.54 72.136) (end 129.54 72.898) (width 0.1) (layer "F.Cu") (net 16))
 (segment (start 132.08 64.96) (end 129.3 64.96) (width 0.1) (layer "F.Cu") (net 16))
 (segment (start 129.859999 71.816001) (end 129.54 72.136) (width 0.1) (layer "F.Cu") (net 16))
 (segment (start 130.505 68.652549) (end 129.859999 69.29755) (width 0.1) (layer "F.Cu") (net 16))
 (segment (start 129.3 64.96) (end 128.475 64.135) (width 0.1) (layer "F.Cu") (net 16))
 (segment (start 132.08 64.96) (end 130.505 66.535) (width 0.1) (layer "F.Cu") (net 16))
 (segment (start 119.81 63.5) (end 120.65 63.5) (width 0.1) (layer "F.Cu") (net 18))
 (segment (start 128.016 67.31) (end 128.73355 66.59245) (width 0.1) (layer "F.Cu") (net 18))
 (segment (start 123.952 65.278) (end 125.984 67.31) (width 0.1) (layer "F.Cu") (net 18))
 (segment (start 128.73355 66.59245) (end 129.859999 66.59245) (width 0.1) (layer "F.Cu") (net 18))
 (segment (start 125.984 67.31) (end 128.016 67.31) (width 0.1) (layer "F.Cu") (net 18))
 (segment (start 120.65 63.5) (end 122.428 65.278) (width 0.1) (layer "F.Cu") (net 18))
 (segment (start 122.428 65.278) (end 123.952 65.278) (width 0.1) (layer "F.Cu") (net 18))
 (segment (start 132.08 62.86) (end 132.08 60.445299) (width 0.1) (layer "F.Cu") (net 17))
 (segment (start 132.08 60.445299) (end 131.815 60.180299) (width 0.1) (layer "F.Cu") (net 17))
 (segment (start 128.658602 61.468) (end 128.778 61.468) (width 0.1) (layer "F.Cu") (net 30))
 (segment (start 127.790001 60.599399) (end 128.658602 61.468) (width 0.1) (layer "F.Cu") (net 30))
 (segment (start 127.790001 60.180299) (end 127.790001 60.599399) (width 0.1) (layer "F.Cu") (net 30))
 (via (at 128.778 61.468) (size 0.8) (drill 0.4) (layers "F.Cu" "B.Cu") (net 30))
 (segment (start 128.778 61.976) (end 127.809 62.945) (width 0.1) (layer "B.Cu") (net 30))
 (segment (start 127.809 62.945) (end 127.635 62.945) (width 0.1) (layer "B.Cu") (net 30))
 (segment (start 128.778 61.468) (end 128.778 61.976) (width 0.1) (layer "B.Cu") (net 30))
 (segment (start 130.79 61.575) (end 130.81 61.595) (width 0.1) (layer "F.Cu") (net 22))
 (segment (start 130.79 60.180299) (end 130.79 61.575) (width 0.1) (layer "F.Cu") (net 22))
 (via (at 130.81 61.595) (size 0.8) (drill 0.4) (layers "F.Cu" "B.Cu") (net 22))
 (segment (start 130.81 61.595) (end 132.08 62.865) (width 0.1) (layer "B.Cu") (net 22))
 (segment (start 132.08 62.865) (end 132.08 62.945) (width 0.1) (layer "B.Cu") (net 22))
 (segment (start 131.760001 69.29755) (end 131.760001 71.562001) (width 0.1) (layer "F.Cu") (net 19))
 (segment (start 131.760001 71.562001) (end 132.08 71.882) (width 0.1) (layer "F.Cu") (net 19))
 (segment (start 132.08 72.71) (end 131.13 73.66) (width 0.1) (layer "F.Cu") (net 19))
 (segment (start 132.08 71.882) (end 132.08 72.71) (width 0.1) (layer "F.Cu") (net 19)))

